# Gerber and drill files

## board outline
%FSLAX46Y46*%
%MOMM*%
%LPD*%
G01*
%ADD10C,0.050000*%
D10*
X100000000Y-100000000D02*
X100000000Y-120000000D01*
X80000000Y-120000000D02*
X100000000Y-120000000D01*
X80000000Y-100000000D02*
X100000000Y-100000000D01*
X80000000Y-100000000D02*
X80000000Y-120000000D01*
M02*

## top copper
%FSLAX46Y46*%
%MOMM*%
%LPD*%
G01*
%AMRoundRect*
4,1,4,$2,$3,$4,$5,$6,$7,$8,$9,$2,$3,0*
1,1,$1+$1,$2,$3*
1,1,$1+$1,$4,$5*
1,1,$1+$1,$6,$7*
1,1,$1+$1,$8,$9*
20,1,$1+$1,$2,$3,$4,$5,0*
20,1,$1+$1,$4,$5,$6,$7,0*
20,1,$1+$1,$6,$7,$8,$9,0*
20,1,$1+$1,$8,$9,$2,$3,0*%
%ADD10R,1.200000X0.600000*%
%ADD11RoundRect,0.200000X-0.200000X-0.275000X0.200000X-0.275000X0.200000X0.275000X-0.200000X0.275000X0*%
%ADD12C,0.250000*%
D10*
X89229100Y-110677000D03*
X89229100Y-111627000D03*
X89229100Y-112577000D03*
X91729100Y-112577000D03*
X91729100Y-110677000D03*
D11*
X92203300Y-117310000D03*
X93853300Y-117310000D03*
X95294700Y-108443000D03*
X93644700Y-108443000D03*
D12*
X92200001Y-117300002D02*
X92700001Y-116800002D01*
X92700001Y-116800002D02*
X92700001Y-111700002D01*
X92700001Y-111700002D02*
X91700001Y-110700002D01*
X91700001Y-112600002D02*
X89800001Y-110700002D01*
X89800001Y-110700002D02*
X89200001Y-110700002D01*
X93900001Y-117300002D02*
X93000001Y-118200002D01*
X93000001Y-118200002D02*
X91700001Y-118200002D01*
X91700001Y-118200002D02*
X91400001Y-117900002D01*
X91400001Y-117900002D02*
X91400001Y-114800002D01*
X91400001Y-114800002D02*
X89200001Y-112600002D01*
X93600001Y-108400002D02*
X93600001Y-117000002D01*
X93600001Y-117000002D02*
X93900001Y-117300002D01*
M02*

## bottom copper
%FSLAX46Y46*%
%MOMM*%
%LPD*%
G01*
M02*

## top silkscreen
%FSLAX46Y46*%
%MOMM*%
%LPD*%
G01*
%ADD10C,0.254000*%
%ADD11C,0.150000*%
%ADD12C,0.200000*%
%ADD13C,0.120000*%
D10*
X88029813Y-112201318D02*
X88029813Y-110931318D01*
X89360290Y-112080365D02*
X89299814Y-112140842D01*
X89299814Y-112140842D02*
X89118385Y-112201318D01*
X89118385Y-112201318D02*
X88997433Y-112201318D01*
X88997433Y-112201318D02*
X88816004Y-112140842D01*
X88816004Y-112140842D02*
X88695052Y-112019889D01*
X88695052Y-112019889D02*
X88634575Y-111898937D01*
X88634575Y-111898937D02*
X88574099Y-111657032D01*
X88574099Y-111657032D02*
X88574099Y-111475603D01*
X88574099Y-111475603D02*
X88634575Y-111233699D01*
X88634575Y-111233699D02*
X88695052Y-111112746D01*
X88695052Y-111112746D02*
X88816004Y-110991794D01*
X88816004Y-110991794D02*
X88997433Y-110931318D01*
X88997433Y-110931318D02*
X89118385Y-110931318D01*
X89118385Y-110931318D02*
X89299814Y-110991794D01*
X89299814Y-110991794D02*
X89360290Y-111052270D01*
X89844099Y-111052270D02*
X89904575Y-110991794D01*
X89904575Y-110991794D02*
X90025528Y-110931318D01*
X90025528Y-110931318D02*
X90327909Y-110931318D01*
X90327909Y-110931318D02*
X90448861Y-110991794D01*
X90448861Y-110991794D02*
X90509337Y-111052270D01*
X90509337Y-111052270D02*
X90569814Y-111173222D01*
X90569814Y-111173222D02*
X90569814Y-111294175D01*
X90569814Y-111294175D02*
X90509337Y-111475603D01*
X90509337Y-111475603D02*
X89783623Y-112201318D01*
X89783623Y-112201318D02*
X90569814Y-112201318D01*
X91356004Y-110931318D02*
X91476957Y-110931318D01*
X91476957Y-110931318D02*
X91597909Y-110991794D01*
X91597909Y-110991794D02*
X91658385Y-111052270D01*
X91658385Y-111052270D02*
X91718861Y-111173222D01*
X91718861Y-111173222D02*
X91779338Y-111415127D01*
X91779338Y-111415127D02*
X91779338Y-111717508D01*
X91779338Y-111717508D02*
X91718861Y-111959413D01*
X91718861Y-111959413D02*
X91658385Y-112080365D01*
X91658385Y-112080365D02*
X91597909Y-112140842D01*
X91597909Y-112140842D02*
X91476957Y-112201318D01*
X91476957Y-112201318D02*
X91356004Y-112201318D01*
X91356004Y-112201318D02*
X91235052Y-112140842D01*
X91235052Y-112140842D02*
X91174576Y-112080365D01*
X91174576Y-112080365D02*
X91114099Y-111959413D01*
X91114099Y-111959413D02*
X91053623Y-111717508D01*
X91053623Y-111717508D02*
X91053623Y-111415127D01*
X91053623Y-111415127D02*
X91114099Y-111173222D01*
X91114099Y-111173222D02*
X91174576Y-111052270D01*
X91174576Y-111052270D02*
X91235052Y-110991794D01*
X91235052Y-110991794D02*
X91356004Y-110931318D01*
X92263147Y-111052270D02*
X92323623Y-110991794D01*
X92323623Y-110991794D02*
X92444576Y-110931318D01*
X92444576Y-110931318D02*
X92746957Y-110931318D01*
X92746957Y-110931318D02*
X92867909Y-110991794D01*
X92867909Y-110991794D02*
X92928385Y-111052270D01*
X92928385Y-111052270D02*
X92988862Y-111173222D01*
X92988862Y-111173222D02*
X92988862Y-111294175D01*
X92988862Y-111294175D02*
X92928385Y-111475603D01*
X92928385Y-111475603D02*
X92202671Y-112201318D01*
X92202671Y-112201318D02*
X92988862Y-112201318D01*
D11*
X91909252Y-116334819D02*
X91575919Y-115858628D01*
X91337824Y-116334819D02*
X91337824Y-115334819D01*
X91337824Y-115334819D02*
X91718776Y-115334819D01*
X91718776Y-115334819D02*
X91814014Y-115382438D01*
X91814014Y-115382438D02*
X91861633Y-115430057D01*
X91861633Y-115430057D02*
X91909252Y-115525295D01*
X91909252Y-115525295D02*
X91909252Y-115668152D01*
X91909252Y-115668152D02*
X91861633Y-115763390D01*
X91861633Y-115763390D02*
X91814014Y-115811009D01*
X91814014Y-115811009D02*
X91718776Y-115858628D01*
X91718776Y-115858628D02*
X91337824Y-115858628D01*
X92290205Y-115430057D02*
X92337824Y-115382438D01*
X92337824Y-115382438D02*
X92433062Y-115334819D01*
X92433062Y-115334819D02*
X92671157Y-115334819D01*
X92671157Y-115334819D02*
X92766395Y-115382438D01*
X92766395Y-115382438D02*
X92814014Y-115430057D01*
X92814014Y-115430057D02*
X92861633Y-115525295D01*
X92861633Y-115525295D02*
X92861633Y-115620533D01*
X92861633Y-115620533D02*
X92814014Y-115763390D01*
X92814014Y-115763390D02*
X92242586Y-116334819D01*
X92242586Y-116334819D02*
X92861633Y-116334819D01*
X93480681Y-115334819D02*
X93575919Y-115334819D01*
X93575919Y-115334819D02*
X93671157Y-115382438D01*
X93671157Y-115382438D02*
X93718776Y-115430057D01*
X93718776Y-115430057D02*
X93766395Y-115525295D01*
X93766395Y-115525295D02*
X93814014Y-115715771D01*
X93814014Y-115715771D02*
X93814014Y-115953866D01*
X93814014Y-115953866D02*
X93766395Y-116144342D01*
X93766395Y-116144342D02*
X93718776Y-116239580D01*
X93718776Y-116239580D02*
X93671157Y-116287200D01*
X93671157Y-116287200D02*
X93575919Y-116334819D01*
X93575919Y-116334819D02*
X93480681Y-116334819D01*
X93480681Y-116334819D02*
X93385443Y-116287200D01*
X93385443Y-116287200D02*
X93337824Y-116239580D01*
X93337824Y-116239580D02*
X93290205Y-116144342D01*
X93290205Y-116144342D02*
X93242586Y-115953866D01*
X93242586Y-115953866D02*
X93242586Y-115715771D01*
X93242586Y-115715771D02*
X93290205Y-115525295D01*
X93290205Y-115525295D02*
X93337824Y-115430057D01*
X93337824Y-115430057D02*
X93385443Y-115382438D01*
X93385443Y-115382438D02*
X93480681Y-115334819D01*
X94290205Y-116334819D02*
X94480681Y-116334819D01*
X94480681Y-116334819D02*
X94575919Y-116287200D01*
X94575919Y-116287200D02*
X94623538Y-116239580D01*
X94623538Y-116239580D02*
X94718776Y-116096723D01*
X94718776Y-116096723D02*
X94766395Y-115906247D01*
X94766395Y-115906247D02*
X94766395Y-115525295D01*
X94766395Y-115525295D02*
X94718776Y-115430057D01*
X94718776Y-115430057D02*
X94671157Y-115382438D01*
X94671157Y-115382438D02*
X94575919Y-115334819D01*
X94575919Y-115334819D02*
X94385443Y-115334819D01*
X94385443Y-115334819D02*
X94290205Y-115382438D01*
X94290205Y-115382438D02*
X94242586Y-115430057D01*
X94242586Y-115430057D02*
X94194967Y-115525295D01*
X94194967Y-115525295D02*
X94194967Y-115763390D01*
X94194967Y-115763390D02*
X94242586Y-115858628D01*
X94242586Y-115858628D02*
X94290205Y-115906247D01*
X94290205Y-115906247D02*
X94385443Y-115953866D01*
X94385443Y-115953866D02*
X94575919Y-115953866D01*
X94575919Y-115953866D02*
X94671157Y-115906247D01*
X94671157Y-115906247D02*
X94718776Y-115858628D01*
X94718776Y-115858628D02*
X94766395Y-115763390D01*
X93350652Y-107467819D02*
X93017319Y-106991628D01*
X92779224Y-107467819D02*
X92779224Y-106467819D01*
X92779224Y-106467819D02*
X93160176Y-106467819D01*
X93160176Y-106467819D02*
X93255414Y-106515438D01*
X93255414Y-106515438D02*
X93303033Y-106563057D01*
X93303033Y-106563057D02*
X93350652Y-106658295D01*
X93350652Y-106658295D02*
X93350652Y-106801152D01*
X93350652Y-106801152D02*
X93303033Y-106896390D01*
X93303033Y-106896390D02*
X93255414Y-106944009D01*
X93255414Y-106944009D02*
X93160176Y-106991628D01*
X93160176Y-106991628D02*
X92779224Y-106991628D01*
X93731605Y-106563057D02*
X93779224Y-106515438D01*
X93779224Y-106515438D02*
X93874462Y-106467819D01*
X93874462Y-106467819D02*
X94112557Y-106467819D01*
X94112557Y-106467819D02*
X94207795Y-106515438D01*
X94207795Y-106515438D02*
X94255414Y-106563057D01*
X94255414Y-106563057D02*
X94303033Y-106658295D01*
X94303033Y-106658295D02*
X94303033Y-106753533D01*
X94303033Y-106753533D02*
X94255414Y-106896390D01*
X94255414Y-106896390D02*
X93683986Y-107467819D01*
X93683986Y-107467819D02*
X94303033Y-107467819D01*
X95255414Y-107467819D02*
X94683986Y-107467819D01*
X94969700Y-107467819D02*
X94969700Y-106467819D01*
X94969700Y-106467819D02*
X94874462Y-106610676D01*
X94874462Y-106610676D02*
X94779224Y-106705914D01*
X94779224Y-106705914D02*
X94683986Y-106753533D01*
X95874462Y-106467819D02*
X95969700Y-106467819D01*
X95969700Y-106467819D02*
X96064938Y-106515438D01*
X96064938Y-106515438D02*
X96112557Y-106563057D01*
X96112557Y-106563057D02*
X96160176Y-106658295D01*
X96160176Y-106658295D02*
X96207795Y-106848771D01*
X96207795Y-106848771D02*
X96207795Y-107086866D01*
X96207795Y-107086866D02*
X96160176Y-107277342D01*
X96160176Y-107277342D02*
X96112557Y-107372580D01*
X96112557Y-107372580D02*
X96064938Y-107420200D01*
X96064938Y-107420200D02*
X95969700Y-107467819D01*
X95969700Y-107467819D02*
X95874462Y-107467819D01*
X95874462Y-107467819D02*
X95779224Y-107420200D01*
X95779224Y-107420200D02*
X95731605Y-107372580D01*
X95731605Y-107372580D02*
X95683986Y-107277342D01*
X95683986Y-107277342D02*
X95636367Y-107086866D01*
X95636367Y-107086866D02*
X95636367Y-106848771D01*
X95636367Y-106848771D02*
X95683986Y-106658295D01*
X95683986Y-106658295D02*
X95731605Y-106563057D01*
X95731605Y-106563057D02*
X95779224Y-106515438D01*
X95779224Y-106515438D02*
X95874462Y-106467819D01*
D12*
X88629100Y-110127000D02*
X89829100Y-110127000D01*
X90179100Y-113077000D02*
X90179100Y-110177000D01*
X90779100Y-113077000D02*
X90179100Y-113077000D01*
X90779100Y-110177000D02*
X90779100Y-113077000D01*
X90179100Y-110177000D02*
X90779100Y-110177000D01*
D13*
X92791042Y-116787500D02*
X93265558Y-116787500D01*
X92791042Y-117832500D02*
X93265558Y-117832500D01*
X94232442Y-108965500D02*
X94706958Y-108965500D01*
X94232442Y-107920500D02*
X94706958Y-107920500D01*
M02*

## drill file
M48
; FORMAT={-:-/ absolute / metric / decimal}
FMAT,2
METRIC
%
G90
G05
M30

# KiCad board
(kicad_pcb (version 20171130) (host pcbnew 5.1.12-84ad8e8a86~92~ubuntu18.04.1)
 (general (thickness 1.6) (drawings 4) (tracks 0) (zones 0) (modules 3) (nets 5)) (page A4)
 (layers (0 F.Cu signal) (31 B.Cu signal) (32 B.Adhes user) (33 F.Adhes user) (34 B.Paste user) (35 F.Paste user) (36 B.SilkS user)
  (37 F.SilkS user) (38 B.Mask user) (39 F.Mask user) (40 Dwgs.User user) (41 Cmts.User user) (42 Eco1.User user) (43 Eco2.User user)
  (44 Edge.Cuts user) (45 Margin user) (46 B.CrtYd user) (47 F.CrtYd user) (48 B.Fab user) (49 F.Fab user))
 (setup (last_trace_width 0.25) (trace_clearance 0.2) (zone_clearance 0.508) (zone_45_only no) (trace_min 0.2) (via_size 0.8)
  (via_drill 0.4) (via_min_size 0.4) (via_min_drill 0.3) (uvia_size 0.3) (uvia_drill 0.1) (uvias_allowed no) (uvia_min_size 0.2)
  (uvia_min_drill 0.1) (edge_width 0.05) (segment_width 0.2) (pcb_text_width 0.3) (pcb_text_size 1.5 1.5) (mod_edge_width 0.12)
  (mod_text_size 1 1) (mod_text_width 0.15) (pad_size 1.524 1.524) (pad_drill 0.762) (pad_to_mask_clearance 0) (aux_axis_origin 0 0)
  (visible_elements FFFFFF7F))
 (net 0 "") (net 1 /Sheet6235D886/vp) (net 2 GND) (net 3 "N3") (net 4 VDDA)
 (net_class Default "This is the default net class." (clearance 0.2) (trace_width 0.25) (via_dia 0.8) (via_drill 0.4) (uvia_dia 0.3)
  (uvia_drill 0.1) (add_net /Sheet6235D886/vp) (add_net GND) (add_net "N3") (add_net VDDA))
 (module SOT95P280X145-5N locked (layer F.Cu) (at 90.479100 111.627000)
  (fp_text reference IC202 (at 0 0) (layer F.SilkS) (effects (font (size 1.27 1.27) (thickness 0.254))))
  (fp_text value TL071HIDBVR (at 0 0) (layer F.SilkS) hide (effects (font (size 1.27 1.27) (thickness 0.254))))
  (fp_line (start -1.85 -1.5) (end -0.65 -1.5) (layer F.SilkS) (width 0.2))
  (fp_line (start -0.3 1.45) (end -0.3 -1.45) (layer F.SilkS) (width 0.2))
  (fp_line (start 0.3 1.45) (end -0.3 1.45) (layer F.SilkS) (width 0.2))
  (fp_line (start 0.3 -1.45) (end 0.3 1.45) (layer F.SilkS) (width 0.2))
  (fp_line (start -0.3 -1.45) (end 0.3 -1.45) (layer F.SilkS) (width 0.2))
  (pad 1 smd rect (at -1.25 -0.95 90.000000) (size 0.6 1.2) (layers F.Cu F.Mask F.Paste) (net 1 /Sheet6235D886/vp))
  (pad 2 smd rect (at -1.25 0 90.000000) (size 0.6 1.2) (layers F.Cu F.Mask F.Paste) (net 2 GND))
  (pad 3 smd rect (at -1.25 0.95 90.000000) (size 0.6 1.2) (layers F.Cu F.Mask F.Paste) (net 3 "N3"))
  (pad 4 smd rect (at 1.25 0.95 90.000000) (size 0.6 1.2) (layers F.Cu F.Mask F.Paste) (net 1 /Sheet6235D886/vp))
  (pad 5 smd rect (at 1.25 -0.95 90.000000) (size 0.6 1.2) (layers F.Cu F.Mask F.Paste) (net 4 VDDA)))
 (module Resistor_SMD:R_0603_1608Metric (layer F.Cu) (at 93.028300 117.310000)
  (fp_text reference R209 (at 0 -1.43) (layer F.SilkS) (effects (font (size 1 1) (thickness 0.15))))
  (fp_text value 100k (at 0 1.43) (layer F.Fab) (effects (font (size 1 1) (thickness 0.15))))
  (fp_line (start -0.237258 -0.5225) (end 0.237258 -0.5225) (layer F.SilkS) (width 0.12))
  (fp_line (start -0.237258 0.5225) (end 0.237258 0.5225) (layer F.SilkS) (width 0.12))
  (pad 1 smd roundrect (at -0.825 0) (size 0.8 0.95) (layers F.Cu F.Mask F.Paste) (roundrect_rratio 0.25) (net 4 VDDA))
  (pad 2 smd roundrect (at 0.825 0) (size 0.8 0.95) (layers F.Cu F.Mask F.Paste) (roundrect_rratio 0.25) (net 3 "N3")))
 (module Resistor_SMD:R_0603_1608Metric (layer F.Cu) (at 94.469700 108.443000)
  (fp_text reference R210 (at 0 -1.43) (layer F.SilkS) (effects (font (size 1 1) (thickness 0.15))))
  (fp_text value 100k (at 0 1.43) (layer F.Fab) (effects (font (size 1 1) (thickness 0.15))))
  (fp_line (start -0.237258 0.5225) (end 0.237258 0.5225) (layer F.SilkS) (width 0.12))
  (fp_line (start -0.237258 -0.5225) (end 0.237258 -0.5225) (layer F.SilkS) (width 0.12))
  (pad 2 smd roundrect (at 0.825 0) (size 0.8 0.95) (layers F.Cu F.Mask F.Paste) (roundrect_rratio 0.25) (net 2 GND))
  (pad 1 smd roundrect (at -0.825 0) (size 0.8 0.95) (layers F.Cu F.Mask F.Paste) (roundrect_rratio 0.25) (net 3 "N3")))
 (gr_line (start 100 100) (end 100 120) (layer Edge.Cuts) (width 0.05))
 (gr_line (start 80 120) (end 100 120) (layer Edge.Cuts) (width 0.05))
 (gr_line (start 80 100) (end 100 100) (layer Edge.Cuts) (width 0.05))
 (gr_line (start 80 100) (end 80 120) (layer Edge.Cuts) (width 0.05))
 (segment (start 92.200001 117.300002) (end 92.700001 116.800002) (width 0.250000) (layer F.Cu) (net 4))
 (segment (start 92.700001 116.800002) (end 92.700001 111.700002) (width 0.250000) (layer F.Cu) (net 4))
 (segment (start 92.700001 111.700002) (end 91.700001 110.700002) (width 0.250000) (layer F.Cu) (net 4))
 (segment (start 91.700001 112.600002) (end 89.800001 110.700002) (width 0.250000) (layer F.Cu) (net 1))
 (segment (start 89.800001 110.700002) (end 89.200001 110.700002) (width 0.250000) (layer F.Cu) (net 1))
 (segment (start 93.900001 117.300002) (end 93.000001 118.200002) (width 0.250000) (layer F.Cu) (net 3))
 (segment (start 93.000001 118.200002) (end 91.700001 118.200002) (width 0.250000) (layer F.Cu) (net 3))
 (segment (start 91.700001 118.200002) (end 91.400001 117.900002) (width 0.250000) (layer F.Cu) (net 3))
 (segment (start 91.400001 117.900002) (end 91.400001 114.800002) (width 0.250000) (layer F.Cu) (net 3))
 (segment (start 91.400001 114.800002) (end 89.200001 112.600002) (width 0.250000) (layer F.Cu) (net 3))
 (segment (start 93.600001 108.400002) (end 93.600001 117.000002) (width 0.250000) (layer F.Cu) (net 3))
 (segment (start 93.600001 117.000002) (end 93.900001 117.300002) (width 0.250000) (layer F.Cu) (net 3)))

